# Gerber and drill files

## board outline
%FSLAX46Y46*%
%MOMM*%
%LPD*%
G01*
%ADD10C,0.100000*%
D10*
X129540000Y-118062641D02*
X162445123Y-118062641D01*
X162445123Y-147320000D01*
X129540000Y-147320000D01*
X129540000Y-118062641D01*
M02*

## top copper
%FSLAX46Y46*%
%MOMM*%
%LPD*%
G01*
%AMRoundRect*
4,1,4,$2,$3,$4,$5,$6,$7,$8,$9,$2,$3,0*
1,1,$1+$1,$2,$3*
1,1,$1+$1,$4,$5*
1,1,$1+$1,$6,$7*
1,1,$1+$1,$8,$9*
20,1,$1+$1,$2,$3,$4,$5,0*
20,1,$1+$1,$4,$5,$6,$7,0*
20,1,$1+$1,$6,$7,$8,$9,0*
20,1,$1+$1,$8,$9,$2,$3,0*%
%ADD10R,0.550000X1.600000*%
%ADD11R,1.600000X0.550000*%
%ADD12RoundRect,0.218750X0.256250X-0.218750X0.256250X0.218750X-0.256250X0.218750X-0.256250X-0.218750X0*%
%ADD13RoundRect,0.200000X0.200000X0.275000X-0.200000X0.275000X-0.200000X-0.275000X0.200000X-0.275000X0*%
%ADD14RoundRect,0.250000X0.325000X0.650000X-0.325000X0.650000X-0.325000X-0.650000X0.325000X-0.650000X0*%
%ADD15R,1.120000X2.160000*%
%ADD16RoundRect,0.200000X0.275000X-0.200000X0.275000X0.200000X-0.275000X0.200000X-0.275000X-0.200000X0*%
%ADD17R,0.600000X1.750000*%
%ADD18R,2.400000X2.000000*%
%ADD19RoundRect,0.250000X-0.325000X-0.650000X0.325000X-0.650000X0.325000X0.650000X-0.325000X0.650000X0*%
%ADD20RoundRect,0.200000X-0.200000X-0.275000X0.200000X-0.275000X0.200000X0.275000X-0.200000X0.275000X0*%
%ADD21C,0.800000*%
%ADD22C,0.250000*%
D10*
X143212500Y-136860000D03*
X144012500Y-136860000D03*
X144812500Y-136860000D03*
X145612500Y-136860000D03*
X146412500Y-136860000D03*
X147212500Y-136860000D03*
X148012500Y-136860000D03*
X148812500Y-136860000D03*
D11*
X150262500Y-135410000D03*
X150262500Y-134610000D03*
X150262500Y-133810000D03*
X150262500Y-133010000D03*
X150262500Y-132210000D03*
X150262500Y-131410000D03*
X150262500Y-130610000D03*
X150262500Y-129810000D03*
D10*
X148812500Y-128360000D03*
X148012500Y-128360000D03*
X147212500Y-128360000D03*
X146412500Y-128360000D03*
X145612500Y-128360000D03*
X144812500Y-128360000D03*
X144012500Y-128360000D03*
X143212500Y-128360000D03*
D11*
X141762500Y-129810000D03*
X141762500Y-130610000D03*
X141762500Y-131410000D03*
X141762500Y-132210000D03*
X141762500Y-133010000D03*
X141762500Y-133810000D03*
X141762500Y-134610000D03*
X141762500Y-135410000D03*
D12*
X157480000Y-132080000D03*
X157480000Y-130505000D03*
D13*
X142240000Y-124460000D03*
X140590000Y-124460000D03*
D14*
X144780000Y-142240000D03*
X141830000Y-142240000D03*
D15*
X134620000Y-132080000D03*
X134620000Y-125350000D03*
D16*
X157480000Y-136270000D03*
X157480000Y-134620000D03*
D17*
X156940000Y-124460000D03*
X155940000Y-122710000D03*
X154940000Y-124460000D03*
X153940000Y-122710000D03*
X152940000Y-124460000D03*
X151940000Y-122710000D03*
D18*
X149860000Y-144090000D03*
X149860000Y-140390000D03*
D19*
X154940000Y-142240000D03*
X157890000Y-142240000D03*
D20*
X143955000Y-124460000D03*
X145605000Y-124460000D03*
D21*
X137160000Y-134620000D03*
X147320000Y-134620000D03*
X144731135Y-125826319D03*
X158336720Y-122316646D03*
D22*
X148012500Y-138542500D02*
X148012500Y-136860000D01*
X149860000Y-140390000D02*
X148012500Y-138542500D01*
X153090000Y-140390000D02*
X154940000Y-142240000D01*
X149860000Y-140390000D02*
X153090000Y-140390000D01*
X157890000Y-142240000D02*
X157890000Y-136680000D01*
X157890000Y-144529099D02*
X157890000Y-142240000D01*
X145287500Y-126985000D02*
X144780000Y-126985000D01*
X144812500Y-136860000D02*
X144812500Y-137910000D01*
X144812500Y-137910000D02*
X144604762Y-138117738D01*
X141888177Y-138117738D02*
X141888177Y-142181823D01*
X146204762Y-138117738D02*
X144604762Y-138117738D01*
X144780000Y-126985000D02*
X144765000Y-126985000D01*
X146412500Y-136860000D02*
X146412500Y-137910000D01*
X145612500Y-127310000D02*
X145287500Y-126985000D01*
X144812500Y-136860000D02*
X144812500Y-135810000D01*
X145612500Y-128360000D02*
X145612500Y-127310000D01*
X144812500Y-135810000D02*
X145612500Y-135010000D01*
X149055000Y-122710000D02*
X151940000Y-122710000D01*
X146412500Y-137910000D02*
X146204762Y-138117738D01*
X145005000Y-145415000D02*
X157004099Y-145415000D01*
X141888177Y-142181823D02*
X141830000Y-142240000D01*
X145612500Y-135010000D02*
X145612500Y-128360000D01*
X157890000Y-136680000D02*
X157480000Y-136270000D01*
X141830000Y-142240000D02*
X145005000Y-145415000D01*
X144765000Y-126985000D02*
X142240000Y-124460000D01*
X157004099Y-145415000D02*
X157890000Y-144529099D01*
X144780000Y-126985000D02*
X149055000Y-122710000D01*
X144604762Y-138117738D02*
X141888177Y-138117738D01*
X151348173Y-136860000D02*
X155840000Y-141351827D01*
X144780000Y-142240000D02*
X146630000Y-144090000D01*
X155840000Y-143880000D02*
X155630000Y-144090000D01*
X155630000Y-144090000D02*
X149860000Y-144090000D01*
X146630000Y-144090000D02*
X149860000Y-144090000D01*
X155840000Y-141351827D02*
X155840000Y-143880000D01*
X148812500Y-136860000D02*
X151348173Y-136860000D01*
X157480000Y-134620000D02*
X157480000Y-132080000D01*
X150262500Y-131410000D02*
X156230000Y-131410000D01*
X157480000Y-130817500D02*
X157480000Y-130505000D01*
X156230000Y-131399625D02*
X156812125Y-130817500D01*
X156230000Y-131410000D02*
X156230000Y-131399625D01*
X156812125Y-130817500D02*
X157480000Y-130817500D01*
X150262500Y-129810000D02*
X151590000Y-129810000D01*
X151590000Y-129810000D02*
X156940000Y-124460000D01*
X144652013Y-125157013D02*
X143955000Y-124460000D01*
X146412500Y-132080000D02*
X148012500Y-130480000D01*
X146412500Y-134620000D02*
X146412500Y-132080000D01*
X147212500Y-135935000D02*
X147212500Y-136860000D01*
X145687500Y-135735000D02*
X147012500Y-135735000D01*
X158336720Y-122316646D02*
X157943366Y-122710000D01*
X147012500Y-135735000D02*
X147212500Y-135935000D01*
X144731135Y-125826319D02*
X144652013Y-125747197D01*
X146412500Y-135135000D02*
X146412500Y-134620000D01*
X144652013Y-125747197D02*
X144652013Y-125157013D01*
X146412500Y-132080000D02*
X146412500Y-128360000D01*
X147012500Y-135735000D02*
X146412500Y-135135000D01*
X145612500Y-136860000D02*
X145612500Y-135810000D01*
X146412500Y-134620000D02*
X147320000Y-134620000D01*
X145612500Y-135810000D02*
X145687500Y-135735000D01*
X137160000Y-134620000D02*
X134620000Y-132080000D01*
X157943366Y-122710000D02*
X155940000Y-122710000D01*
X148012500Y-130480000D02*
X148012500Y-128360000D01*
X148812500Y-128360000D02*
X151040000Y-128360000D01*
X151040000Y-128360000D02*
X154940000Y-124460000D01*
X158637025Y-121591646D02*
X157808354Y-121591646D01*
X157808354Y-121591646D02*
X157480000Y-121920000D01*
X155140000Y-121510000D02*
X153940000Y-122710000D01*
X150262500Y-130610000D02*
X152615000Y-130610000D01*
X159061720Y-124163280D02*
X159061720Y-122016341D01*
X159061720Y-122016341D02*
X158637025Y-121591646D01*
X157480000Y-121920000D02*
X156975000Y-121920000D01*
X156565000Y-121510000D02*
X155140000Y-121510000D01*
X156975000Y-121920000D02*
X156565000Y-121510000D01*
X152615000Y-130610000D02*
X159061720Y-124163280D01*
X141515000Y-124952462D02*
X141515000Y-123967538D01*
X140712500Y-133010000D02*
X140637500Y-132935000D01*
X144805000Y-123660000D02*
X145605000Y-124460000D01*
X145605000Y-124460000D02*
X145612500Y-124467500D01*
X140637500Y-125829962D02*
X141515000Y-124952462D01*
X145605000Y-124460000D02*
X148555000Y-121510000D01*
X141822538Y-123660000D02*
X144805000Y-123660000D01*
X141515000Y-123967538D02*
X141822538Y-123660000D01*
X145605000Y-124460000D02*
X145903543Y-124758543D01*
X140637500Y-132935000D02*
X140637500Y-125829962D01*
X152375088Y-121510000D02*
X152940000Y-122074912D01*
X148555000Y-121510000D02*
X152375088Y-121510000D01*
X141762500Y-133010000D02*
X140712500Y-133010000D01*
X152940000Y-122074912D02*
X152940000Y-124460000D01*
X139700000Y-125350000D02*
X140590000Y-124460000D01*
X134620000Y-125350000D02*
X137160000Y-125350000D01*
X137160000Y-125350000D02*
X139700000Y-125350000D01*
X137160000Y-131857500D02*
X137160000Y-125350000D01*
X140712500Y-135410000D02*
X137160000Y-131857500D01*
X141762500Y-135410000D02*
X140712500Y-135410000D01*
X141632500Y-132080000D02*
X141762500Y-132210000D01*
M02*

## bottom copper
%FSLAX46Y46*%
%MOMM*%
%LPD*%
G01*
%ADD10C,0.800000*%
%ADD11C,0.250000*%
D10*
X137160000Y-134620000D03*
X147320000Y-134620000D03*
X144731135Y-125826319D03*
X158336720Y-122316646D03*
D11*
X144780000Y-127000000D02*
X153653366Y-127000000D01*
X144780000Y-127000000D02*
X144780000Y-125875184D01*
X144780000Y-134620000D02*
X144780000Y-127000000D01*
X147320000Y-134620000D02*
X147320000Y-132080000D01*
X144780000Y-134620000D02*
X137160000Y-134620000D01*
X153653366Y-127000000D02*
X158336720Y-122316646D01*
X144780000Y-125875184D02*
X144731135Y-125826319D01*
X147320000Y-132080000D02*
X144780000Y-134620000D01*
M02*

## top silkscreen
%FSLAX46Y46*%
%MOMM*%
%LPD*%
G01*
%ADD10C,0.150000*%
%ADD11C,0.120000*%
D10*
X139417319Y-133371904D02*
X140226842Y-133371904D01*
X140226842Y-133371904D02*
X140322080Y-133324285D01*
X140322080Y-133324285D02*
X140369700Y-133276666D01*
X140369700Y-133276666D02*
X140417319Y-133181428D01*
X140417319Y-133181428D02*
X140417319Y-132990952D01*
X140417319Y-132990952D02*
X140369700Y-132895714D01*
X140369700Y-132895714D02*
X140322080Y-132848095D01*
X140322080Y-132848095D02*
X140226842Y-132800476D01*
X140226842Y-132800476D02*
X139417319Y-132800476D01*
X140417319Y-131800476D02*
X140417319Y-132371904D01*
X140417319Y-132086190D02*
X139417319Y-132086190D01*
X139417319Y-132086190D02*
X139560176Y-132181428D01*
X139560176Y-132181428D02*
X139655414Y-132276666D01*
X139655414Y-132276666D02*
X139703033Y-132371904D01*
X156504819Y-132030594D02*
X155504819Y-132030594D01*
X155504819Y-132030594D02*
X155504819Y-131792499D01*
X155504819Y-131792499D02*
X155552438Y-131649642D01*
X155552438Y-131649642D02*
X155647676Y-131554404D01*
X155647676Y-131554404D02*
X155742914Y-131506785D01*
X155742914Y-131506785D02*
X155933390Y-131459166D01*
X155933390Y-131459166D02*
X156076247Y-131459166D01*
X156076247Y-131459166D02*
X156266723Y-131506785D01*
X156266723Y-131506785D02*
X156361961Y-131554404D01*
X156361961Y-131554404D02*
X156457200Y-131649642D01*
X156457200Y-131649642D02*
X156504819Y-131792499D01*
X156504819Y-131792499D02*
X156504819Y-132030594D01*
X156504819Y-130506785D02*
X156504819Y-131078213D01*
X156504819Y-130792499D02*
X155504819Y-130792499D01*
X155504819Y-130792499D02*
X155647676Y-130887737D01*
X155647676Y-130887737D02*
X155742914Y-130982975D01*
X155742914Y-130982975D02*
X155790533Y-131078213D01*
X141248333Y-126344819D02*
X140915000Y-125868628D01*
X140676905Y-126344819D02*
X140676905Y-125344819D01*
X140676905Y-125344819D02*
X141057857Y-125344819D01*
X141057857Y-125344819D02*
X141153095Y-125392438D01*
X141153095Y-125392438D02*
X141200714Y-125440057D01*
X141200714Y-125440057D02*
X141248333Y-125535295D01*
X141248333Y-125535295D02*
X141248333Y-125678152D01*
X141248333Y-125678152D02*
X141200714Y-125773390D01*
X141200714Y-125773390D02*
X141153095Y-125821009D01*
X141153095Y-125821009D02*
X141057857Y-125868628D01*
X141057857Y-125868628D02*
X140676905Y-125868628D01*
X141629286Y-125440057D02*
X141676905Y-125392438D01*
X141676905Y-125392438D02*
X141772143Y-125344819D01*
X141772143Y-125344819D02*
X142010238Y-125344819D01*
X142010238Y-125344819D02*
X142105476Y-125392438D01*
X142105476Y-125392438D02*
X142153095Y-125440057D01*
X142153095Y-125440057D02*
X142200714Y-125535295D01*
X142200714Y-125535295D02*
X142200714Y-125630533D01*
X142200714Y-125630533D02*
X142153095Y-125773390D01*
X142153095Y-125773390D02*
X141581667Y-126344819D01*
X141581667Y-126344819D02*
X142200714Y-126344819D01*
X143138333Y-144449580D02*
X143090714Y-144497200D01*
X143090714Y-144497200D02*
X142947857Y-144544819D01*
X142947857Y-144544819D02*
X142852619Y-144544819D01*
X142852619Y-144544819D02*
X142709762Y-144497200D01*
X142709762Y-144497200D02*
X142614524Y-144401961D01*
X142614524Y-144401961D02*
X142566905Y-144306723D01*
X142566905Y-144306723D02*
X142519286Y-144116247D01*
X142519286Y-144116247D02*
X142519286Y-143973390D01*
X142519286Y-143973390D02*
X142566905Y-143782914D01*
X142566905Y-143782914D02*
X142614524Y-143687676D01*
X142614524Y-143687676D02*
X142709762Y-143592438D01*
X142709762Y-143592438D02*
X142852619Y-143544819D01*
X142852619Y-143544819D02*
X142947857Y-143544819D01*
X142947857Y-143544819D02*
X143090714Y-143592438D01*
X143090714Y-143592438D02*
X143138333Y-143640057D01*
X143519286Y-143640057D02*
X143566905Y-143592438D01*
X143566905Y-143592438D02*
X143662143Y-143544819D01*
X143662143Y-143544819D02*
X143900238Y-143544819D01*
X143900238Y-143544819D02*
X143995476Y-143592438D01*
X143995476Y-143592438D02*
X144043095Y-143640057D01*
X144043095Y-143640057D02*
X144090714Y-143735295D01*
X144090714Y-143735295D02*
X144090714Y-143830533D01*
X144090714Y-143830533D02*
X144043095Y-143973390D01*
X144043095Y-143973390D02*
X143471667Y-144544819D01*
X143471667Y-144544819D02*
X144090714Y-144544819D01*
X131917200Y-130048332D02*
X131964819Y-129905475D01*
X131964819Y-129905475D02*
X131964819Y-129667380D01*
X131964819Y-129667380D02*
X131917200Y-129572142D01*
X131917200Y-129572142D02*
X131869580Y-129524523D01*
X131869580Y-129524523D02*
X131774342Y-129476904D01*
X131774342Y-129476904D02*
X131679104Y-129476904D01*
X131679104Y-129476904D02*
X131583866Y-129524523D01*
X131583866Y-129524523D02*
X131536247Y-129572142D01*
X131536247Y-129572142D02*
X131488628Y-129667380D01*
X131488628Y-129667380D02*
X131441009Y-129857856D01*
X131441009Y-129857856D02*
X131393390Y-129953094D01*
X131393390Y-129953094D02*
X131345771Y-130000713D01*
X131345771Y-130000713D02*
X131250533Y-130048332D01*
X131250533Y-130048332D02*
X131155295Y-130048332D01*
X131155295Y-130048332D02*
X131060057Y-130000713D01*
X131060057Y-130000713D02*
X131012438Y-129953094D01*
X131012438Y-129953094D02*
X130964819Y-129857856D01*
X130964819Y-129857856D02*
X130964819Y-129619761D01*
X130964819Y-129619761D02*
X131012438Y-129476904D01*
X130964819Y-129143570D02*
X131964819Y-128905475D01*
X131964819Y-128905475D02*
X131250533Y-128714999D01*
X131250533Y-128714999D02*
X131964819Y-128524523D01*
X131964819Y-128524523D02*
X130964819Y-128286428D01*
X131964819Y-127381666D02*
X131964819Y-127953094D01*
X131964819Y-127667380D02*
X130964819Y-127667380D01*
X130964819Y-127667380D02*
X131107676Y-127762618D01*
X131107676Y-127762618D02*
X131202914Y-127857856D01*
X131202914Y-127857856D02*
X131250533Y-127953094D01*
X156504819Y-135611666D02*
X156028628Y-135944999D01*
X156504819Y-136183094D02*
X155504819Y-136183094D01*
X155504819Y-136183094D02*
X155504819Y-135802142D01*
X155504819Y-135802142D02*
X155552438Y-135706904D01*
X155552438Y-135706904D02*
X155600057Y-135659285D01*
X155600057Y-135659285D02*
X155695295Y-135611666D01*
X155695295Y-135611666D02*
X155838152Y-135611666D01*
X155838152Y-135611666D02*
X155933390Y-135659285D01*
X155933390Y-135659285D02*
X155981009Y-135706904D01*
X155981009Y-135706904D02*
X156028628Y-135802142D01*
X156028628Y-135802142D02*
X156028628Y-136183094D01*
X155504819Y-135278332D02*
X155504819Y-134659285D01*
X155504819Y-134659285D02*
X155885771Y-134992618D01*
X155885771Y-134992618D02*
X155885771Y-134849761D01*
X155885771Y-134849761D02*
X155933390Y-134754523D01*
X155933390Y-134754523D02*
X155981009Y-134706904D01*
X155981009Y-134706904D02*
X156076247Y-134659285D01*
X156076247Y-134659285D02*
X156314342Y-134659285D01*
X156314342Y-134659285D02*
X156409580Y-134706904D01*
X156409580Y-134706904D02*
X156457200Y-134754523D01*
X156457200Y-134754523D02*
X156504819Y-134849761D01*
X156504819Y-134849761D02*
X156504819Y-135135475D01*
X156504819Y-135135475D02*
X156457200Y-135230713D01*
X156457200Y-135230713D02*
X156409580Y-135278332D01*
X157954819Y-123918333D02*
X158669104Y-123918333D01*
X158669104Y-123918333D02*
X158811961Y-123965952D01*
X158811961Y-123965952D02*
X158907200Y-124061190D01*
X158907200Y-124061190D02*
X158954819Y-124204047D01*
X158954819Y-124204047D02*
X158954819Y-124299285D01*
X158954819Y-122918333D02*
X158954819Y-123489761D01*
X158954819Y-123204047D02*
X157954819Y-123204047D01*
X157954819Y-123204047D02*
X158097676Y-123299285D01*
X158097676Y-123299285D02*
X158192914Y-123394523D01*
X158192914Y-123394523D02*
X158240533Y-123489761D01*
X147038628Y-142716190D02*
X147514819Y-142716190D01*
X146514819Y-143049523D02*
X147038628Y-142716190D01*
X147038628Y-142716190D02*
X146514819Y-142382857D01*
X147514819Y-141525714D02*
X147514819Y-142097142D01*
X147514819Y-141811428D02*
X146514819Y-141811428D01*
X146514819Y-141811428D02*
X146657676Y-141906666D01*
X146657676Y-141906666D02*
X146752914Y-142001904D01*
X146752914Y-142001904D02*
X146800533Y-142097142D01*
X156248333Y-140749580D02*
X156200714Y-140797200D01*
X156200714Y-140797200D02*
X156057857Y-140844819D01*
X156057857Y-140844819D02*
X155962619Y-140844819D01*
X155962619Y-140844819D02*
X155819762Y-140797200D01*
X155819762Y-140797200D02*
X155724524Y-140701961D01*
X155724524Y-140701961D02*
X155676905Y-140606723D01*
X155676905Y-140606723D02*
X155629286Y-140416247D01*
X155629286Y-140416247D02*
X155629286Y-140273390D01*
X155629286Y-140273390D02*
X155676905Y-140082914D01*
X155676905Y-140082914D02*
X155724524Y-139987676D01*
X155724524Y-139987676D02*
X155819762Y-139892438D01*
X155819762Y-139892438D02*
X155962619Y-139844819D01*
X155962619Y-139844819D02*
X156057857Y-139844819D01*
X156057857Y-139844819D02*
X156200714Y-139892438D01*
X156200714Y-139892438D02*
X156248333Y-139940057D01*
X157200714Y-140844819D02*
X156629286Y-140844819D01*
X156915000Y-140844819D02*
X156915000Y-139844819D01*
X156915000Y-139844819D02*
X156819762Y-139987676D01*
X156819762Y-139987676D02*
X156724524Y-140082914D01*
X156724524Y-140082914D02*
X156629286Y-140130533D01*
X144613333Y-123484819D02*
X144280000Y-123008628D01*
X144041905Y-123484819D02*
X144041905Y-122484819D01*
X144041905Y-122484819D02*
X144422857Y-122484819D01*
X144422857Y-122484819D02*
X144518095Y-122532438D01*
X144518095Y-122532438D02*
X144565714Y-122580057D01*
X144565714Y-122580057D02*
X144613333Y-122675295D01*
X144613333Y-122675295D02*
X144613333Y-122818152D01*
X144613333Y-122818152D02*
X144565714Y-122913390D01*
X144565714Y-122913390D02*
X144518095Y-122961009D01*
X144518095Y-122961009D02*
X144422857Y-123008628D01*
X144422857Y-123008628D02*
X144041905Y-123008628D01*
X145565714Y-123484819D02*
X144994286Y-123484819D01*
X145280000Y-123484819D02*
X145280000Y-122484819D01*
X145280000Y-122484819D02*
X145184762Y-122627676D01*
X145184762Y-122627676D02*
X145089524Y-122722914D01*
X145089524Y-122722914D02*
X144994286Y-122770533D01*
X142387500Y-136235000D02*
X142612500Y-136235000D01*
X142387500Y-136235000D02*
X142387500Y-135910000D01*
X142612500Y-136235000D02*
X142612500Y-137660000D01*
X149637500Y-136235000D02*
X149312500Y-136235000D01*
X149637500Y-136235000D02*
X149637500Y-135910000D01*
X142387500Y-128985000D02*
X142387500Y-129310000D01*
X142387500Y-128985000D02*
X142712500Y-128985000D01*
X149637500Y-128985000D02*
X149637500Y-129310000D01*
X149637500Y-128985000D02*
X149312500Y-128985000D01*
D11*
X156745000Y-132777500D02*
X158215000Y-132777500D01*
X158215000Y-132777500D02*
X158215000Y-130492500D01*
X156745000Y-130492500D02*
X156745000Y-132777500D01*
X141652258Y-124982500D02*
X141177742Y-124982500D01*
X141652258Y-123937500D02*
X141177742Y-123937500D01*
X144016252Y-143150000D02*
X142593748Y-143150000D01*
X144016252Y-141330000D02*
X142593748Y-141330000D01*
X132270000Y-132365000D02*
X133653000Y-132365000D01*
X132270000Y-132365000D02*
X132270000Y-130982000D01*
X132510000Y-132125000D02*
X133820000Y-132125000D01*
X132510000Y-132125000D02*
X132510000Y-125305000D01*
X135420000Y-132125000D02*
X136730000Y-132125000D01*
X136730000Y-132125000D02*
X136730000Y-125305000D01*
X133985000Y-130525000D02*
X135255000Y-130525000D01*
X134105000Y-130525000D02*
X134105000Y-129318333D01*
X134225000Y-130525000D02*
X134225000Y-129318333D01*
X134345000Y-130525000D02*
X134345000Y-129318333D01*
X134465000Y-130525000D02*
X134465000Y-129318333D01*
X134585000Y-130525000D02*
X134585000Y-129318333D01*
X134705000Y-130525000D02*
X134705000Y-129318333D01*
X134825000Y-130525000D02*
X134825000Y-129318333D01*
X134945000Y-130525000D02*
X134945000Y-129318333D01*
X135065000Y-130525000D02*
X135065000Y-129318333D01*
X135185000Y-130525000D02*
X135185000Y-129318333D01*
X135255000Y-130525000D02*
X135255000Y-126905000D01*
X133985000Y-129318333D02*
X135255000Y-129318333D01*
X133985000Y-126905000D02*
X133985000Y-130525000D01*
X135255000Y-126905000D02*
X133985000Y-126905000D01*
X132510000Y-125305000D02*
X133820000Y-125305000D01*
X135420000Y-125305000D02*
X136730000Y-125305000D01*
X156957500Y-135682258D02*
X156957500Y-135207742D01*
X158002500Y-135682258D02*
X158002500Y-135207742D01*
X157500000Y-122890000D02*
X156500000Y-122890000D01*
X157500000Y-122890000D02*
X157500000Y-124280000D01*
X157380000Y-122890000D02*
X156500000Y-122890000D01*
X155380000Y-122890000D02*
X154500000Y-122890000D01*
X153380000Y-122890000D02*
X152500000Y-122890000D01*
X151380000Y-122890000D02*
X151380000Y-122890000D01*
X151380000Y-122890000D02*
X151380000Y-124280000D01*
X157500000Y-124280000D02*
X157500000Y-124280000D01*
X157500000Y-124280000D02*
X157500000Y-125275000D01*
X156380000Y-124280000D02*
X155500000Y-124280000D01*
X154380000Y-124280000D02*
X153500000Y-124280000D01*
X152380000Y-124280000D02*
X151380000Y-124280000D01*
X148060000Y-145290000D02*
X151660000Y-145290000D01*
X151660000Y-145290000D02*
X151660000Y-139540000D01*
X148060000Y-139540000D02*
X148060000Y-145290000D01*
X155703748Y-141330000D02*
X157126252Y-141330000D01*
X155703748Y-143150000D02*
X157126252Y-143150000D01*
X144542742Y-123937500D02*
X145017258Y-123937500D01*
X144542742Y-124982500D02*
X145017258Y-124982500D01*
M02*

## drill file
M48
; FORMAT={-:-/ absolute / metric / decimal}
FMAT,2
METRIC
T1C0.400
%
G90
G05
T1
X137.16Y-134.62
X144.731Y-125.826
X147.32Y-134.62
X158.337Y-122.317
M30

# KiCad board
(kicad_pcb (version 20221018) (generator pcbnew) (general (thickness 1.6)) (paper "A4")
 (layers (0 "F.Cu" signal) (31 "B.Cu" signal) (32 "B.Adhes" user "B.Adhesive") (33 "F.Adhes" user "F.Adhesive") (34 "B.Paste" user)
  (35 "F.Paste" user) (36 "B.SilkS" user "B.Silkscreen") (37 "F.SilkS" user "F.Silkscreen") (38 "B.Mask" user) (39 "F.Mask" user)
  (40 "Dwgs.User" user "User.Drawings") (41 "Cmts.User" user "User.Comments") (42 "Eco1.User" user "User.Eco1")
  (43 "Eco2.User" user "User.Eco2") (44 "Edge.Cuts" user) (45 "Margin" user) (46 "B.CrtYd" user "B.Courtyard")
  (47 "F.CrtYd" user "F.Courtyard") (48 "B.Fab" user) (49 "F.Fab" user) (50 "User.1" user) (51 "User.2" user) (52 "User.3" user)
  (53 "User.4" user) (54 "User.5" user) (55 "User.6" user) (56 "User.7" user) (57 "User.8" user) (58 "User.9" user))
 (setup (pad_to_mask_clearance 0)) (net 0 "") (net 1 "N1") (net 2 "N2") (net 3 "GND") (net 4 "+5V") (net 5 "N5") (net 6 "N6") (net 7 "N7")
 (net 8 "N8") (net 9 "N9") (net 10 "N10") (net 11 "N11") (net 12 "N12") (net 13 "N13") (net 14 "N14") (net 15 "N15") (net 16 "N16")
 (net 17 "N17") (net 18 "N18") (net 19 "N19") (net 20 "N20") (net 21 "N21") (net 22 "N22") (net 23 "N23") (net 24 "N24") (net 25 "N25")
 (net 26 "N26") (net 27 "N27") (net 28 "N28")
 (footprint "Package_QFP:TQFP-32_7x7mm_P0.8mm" (layer "F.Cu") (at 146.0125 132.61 90)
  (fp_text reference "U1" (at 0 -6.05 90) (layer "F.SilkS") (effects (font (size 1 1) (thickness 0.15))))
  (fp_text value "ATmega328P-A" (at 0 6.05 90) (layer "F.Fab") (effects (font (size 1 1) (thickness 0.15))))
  (fp_line (start -3.625 -3.625) (end -3.625 -3.4) (stroke (width 0.15) (type solid)) (layer "F.SilkS"))
  (fp_line (start -3.625 -3.625) (end -3.3 -3.625) (stroke (width 0.15) (type solid)) (layer "F.SilkS"))
  (fp_line (start -3.625 -3.4) (end -5.05 -3.4) (stroke (width 0.15) (type solid)) (layer "F.SilkS"))
  (fp_line (start -3.625 3.625) (end -3.625 3.3) (stroke (width 0.15) (type solid)) (layer "F.SilkS"))
  (fp_line (start -3.625 3.625) (end -3.3 3.625) (stroke (width 0.15) (type solid)) (layer "F.SilkS"))
  (fp_line (start 3.625 -3.625) (end 3.3 -3.625) (stroke (width 0.15) (type solid)) (layer "F.SilkS"))
  (fp_line (start 3.625 -3.625) (end 3.625 -3.3) (stroke (width 0.15) (type solid)) (layer "F.SilkS"))
  (fp_line (start 3.625 3.625) (end 3.3 3.625) (stroke (width 0.15) (type solid)) (layer "F.SilkS"))
  (fp_line (start 3.625 3.625) (end 3.625 3.3) (stroke (width 0.15) (type solid)) (layer "F.SilkS"))
  (pad "1" smd rect (at -4.25 -2.8 90) (size 1.6 0.55) (layers "F.Cu" "F.Paste" "F.Mask") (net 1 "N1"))
  (pad "2" smd rect (at -4.25 -2 90) (size 1.6 0.55) (layers "F.Cu" "F.Paste" "F.Mask") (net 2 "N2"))
  (pad "3" smd rect (at -4.25 -1.2 90) (size 1.6 0.55) (layers "F.Cu" "F.Paste" "F.Mask") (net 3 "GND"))
  (pad "4" smd rect (at -4.25 -0.4 90) (size 1.6 0.55) (layers "F.Cu" "F.Paste" "F.Mask") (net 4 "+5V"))
  (pad "5" smd rect (at -4.25 0.4 90) (size 1.6 0.55) (layers "F.Cu" "F.Paste" "F.Mask") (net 3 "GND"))
  (pad "6" smd rect (at -4.25 1.2 90) (size 1.6 0.55) (layers "F.Cu" "F.Paste" "F.Mask") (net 4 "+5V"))
  (pad "7" smd rect (at -4.25 2 90) (size 1.6 0.55) (layers "F.Cu" "F.Paste" "F.Mask") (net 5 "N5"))
  (pad "8" smd rect (at -4.25 2.8 90) (size 1.6 0.55) (layers "F.Cu" "F.Paste" "F.Mask") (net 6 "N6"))
  (pad "9" smd rect (at -2.8 4.25 180) (size 1.6 0.55) (layers "F.Cu" "F.Paste" "F.Mask") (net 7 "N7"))
  (pad "10" smd rect (at -2 4.25 180) (size 1.6 0.55) (layers "F.Cu" "F.Paste" "F.Mask") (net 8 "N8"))
  (pad "11" smd rect (at -1.2 4.25 180) (size 1.6 0.55) (layers "F.Cu" "F.Paste" "F.Mask") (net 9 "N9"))
  (pad "12" smd rect (at -0.4 4.25 180) (size 1.6 0.55) (layers "F.Cu" "F.Paste" "F.Mask") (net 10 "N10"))
  (pad "13" smd rect (at 0.4 4.25 180) (size 1.6 0.55) (layers "F.Cu" "F.Paste" "F.Mask") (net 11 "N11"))
  (pad "14" smd rect (at 1.2 4.25 180) (size 1.6 0.55) (layers "F.Cu" "F.Paste" "F.Mask") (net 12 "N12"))
  (pad "15" smd rect (at 2 4.25 180) (size 1.6 0.55) (layers "F.Cu" "F.Paste" "F.Mask") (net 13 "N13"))
  (pad "16" smd rect (at 2.8 4.25 180) (size 1.6 0.55) (layers "F.Cu" "F.Paste" "F.Mask") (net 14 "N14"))
  (pad "17" smd rect (at 4.25 2.8 90) (size 1.6 0.55) (layers "F.Cu" "F.Paste" "F.Mask") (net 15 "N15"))
  (pad "18" smd rect (at 4.25 2 90) (size 1.6 0.55) (layers "F.Cu" "F.Paste" "F.Mask") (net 4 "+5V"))
  (pad "19" smd rect (at 4.25 1.2 90) (size 1.6 0.55) (layers "F.Cu" "F.Paste" "F.Mask") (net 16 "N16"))
  (pad "20" smd rect (at 4.25 0.4 90) (size 1.6 0.55) (layers "F.Cu" "F.Paste" "F.Mask") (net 4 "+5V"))
  (pad "21" smd rect (at 4.25 -0.4 90) (size 1.6 0.55) (layers "F.Cu" "F.Paste" "F.Mask") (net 3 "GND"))
  (pad "22" smd rect (at 4.25 -1.2 90) (size 1.6 0.55) (layers "F.Cu" "F.Paste" "F.Mask") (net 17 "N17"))
  (pad "23" smd rect (at 4.25 -2 90) (size 1.6 0.55) (layers "F.Cu" "F.Paste" "F.Mask") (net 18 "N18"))
  (pad "24" smd rect (at 4.25 -2.8 90) (size 1.6 0.55) (layers "F.Cu" "F.Paste" "F.Mask") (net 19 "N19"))
  (pad "25" smd rect (at 2.8 -4.25 180) (size 1.6 0.55) (layers "F.Cu" "F.Paste" "F.Mask") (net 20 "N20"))
  (pad "26" smd rect (at 2 -4.25 180) (size 1.6 0.55) (layers "F.Cu" "F.Paste" "F.Mask") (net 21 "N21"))
  (pad "27" smd rect (at 1.2 -4.25 180) (size 1.6 0.55) (layers "F.Cu" "F.Paste" "F.Mask") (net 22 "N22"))
  (pad "28" smd rect (at 0.4 -4.25 180) (size 1.6 0.55) (layers "F.Cu" "F.Paste" "F.Mask") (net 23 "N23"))
  (pad "29" smd rect (at -0.4 -4.25 180) (size 1.6 0.55) (layers "F.Cu" "F.Paste" "F.Mask") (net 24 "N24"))
  (pad "30" smd rect (at -1.2 -4.25 180) (size 1.6 0.55) (layers "F.Cu" "F.Paste" "F.Mask") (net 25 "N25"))
  (pad "31" smd rect (at -2 -4.25 180) (size 1.6 0.55) (layers "F.Cu" "F.Paste" "F.Mask") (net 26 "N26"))
  (pad "32" smd rect (at -2.8 -4.25 180) (size 1.6 0.55) (layers "F.Cu" "F.Paste" "F.Mask") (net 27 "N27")))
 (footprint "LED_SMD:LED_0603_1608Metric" (layer "F.Cu") (at 157.48 131.2925 90)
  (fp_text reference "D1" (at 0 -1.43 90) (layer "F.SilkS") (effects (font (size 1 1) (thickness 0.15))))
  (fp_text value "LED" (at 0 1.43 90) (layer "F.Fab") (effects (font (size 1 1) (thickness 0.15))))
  (fp_line (start -1.485 -0.735) (end -1.485 0.735) (stroke (width 0.12) (type solid)) (layer "F.SilkS"))
  (fp_line (start -1.485 0.735) (end 0.8 0.735) (stroke (width 0.12) (type solid)) (layer "F.SilkS"))
  (fp_line (start 0.8 -0.735) (end -1.485 -0.735) (stroke (width 0.12) (type solid)) (layer "F.SilkS"))
  (pad "1" smd roundrect (at -0.7875 0 90) (size 0.875 0.95) (layers "F.Cu" "F.Paste" "F.Mask") (roundrect_rratio 0.25) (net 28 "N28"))
  (pad "2" smd roundrect (at 0.7875 0 90) (size 0.875 0.95) (layers "F.Cu" "F.Paste" "F.Mask") (roundrect_rratio 0.25) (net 12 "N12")))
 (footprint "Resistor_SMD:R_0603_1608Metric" (layer "F.Cu") (at 141.415 124.46 180)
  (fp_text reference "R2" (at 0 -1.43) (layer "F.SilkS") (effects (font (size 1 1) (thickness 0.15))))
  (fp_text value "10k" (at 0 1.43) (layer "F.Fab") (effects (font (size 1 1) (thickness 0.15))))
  (fp_line (start -0.237258 -0.5225) (end 0.237258 -0.5225) (stroke (width 0.12) (type solid)) (layer "F.SilkS"))
  (fp_line (start -0.237258 0.5225) (end 0.237258 0.5225) (stroke (width 0.12) (type solid)) (layer "F.SilkS"))
  (pad "1" smd roundrect (at -0.825 0 180) (size 0.8 0.95) (layers "F.Cu" "F.Paste" "F.Mask") (roundrect_rratio 0.25) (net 3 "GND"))
  (pad "2" smd roundrect (at 0.825 0 180) (size 0.8 0.95) (layers "F.Cu" "F.Paste" "F.Mask") (roundrect_rratio 0.25) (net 27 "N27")))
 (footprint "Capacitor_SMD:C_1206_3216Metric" (layer "F.Cu") (at 143.305 142.24 180)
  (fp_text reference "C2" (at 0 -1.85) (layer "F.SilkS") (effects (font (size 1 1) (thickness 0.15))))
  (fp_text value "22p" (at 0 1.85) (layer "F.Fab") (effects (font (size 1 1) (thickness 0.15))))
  (fp_line (start -0.711252 -0.91) (end 0.711252 -0.91) (stroke (width 0.12) (type solid)) (layer "F.SilkS"))
  (fp_line (start -0.711252 0.91) (end 0.711252 0.91) (stroke (width 0.12) (type solid)) (layer "F.SilkS"))
  (pad "1" smd roundrect (at -1.475 0 180) (size 1.15 1.8) (layers "F.Cu" "F.Paste" "F.Mask") (roundrect_rratio 0.2173913043) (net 6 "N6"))
  (pad "2" smd roundrect (at 1.475 0 180) (size 1.15 1.8) (layers "F.Cu" "F.Paste" "F.Mask") (roundrect_rratio 0.2173913043) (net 3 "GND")))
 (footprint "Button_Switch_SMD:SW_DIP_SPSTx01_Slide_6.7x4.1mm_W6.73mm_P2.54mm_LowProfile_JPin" (layer "F.Cu") (at 134.62 128.715 90)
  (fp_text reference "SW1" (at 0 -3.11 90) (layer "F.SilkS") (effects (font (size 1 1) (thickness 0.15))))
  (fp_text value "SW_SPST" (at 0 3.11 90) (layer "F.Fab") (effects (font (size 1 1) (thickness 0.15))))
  (fp_line (start -3.65 -2.35) (end -3.65 -0.967) (stroke (width 0.12) (type solid)) (layer "F.SilkS"))
  (fp_line (start -3.65 -2.35) (end -2.267 -2.35) (stroke (width 0.12) (type solid)) (layer "F.SilkS"))
  (fp_line (start -3.41 -2.11) (end -3.41 -0.8) (stroke (width 0.12) (type solid)) (layer "F.SilkS"))
  (fp_line (start -3.41 -2.11) (end 3.41 -2.11) (stroke (width 0.12) (type solid)) (layer "F.SilkS"))
  (fp_line (start -3.41 0.8) (end -3.41 2.11) (stroke (width 0.12) (type solid)) (layer "F.SilkS"))
  (fp_line (start -3.41 2.11) (end 3.41 2.11) (stroke (width 0.12) (type solid)) (layer "F.SilkS"))
  (fp_line (start -1.81 -0.635) (end -1.81 0.635) (stroke (width 0.12) (type solid)) (layer "F.SilkS"))
  (fp_line (start -1.81 -0.515) (end -0.603333 -0.515) (stroke (width 0.12) (type solid)) (layer "F.SilkS"))
  (fp_line (start -1.81 -0.395) (end -0.603333 -0.395) (stroke (width 0.12) (type solid)) (layer "F.SilkS"))
  (fp_line (start -1.81 -0.275) (end -0.603333 -0.275) (stroke (width 0.12) (type solid)) (layer "F.SilkS"))
  (fp_line (start -1.81 -0.155) (end -0.603333 -0.155) (stroke (width 0.12) (type solid)) (layer "F.SilkS"))
  (fp_line (start -1.81 -0.035) (end -0.603333 -0.035) (stroke (width 0.12) (type solid)) (layer "F.SilkS"))
  (fp_line (start -1.81 0.085) (end -0.603333 0.085) (stroke (width 0.12) (type solid)) (layer "F.SilkS"))
  (fp_line (start -1.81 0.205) (end -0.603333 0.205) (stroke (width 0.12) (type solid)) (layer "F.SilkS"))
  (fp_line (start -1.81 0.325) (end -0.603333 0.325) (stroke (width 0.12) (type solid)) (layer "F.SilkS"))
  (fp_line (start -1.81 0.445) (end -0.603333 0.445) (stroke (width 0.12) (type solid)) (layer "F.SilkS"))
  (fp_line (start -1.81 0.565) (end -0.603333 0.565) (stroke (width 0.12) (type solid)) (layer "F.SilkS"))
  (fp_line (start -1.81 0.635) (end 1.81 0.635) (stroke (width 0.12) (type solid)) (layer "F.SilkS"))
  (fp_line (start -0.603333 -0.635) (end -0.603333 0.635) (stroke (width 0.12) (type solid)) (layer "F.SilkS"))
  (fp_line (start 1.81 -0.635) (end -1.81 -0.635) (stroke (width 0.12) (type solid)) (layer "F.SilkS"))
  (fp_line (start 1.81 0.635) (end 1.81 -0.635) (stroke (width 0.12) (type solid)) (layer "F.SilkS"))
  (fp_line (start 3.41 -2.11) (end 3.41 -0.8) (stroke (width 0.12) (type solid)) (layer "F.SilkS"))
  (fp_line (start 3.41 0.8) (end 3.41 2.11) (stroke (width 0.12) (type solid)) (layer "F.SilkS"))
  (pad "1" smd rect (at -3.365 0 90) (size 2.16 1.12) (layers "F.Cu" "F.Paste" "F.Mask") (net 4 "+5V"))
  (pad "2" smd rect (at 3.365 0 90) (size 2.16 1.12) (layers "F.Cu" "F.Paste" "F.Mask") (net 27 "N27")))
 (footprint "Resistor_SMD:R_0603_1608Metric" (layer "F.Cu") (at 157.48 135.445 90)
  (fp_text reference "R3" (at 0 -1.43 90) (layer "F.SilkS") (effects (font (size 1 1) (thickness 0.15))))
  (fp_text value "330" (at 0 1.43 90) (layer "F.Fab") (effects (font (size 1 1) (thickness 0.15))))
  (fp_line (start -0.237258 -0.5225) (end 0.237258 -0.5225) (stroke (width 0.12) (type solid)) (layer "F.SilkS"))
  (fp_line (start -0.237258 0.5225) (end 0.237258 0.5225) (stroke (width 0.12) (type solid)) (layer "F.SilkS"))
  (pad "1" smd roundrect (at -0.825 0 90) (size 0.8 0.95) (layers "F.Cu" "F.Paste" "F.Mask") (roundrect_rratio 0.25) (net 3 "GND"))
  (pad "2" smd roundrect (at 0.825 0 90) (size 0.8 0.95) (layers "F.Cu" "F.Paste" "F.Mask") (roundrect_rratio 0.25) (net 28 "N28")))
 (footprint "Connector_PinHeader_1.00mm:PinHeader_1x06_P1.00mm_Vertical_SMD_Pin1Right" (layer "F.Cu") (at 154.44 123.585 -90)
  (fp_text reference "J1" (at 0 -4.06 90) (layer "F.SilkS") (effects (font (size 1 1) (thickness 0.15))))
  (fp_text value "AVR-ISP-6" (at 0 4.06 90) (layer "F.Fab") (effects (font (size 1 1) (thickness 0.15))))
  (fp_line (start -0.695 -3.06) (end -0.695 -2.06) (stroke (width 0.12) (type solid)) (layer "F.SilkS"))
  (fp_line (start -0.695 -3.06) (end 0.695 -3.06) (stroke (width 0.12) (type solid)) (layer "F.SilkS"))
  (fp_line (start -0.695 -2.94) (end -0.695 -2.06) (stroke (width 0.12) (type solid)) (layer "F.SilkS"))
  (fp_line (start -0.695 -0.94) (end -0.695 -0.06) (stroke (width 0.12) (type solid)) (layer "F.SilkS"))
  (fp_line (start -0.695 1.06) (end -0.695 1.94) (stroke (width 0.12) (type solid)) (layer "F.SilkS"))
  (fp_line (start -0.695 3.06) (end -0.695 3.06) (stroke (width 0.12) (type solid)) (layer "F.SilkS"))
  (fp_line (start -0.695 3.06) (end 0.695 3.06) (stroke (width 0.12) (type solid)) (layer "F.SilkS"))
  (fp_line (start 0.695 -3.06) (end 0.695 -3.06) (stroke (width 0.12) (type solid)) (layer "F.SilkS"))
  (fp_line (start 0.695 -3.06) (end 1.69 -3.06) (stroke (width 0.12) (type solid)) (layer "F.SilkS"))
  (fp_line (start 0.695 -1.94) (end 0.695 -1.06) (stroke (width 0.12) (type solid)) (layer "F.SilkS"))
  (fp_line (start 0.695 0.06) (end 0.695 0.94) (stroke (width 0.12) (type solid)) (layer "F.SilkS"))
  (fp_line (start 0.695 2.06) (end 0.695 3.06) (stroke (width 0.12) (type solid)) (layer "F.SilkS"))
  (pad "1" smd rect (at 0.875 -2.5 270) (size 1.75 0.6) (layers "F.Cu" "F.Paste" "F.Mask") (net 14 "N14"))
  (pad "2" smd rect (at -0.875 -1.5 270) (size 1.75 0.6) (layers "F.Cu" "F.Paste" "F.Mask") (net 4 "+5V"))
  (pad "3" smd rect (at 0.875 -0.5 270) (size 1.75 0.6) (layers "F.Cu" "F.Paste" "F.Mask") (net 15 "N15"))
  (pad "4" smd rect (at -0.875 0.5 270) (size 1.75 0.6) (layers "F.Cu" "F.Paste" "F.Mask") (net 13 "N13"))
  (pad "5" smd rect (at 0.875 1.5 270) (size 1.75 0.6) (layers "F.Cu" "F.Paste" "F.Mask") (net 24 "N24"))
  (pad "6" smd rect (at -0.875 2.5 270) (size 1.75 0.6) (layers "F.Cu" "F.Paste" "F.Mask") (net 3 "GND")))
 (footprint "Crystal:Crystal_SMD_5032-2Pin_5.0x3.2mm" (layer "F.Cu") (at 149.86 142.24 90)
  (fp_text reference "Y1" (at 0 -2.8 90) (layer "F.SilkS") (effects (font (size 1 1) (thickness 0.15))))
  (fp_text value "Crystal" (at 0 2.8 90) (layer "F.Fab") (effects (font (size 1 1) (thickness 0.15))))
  (fp_line (start -3.05 -1.8) (end -3.05 1.8) (stroke (width 0.12) (type solid)) (layer "F.SilkS"))
  (fp_line (start -3.05 1.8) (end 2.7 1.8) (stroke (width 0.12) (type solid)) (layer "F.SilkS"))
  (fp_line (start 2.7 -1.8) (end -3.05 -1.8) (stroke (width 0.12) (type solid)) (layer "F.SilkS"))
  (pad "1" smd rect (at -1.85 0 90) (size 2 2.4) (layers "F.Cu" "F.Paste" "F.Mask") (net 6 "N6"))
  (pad "2" smd rect (at 1.85 0 90) (size 2 2.4) (layers "F.Cu" "F.Paste" "F.Mask") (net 5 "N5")))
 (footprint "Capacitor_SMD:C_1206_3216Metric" (layer "F.Cu") (at 156.415 142.24)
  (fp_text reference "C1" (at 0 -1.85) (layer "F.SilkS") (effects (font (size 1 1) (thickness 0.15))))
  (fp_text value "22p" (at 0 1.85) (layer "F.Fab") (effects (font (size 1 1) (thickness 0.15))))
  (fp_line (start -0.711252 -0.91) (end 0.711252 -0.91) (stroke (width 0.12) (type solid)) (layer "F.SilkS"))
  (fp_line (start -0.711252 0.91) (end 0.711252 0.91) (stroke (width 0.12) (type solid)) (layer "F.SilkS"))
  (pad "1" smd roundrect (at -1.475 0) (size 1.15 1.8) (layers "F.Cu" "F.Paste" "F.Mask") (roundrect_rratio 0.2173913043) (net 5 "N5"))
  (pad "2" smd roundrect (at 1.475 0) (size 1.15 1.8) (layers "F.Cu" "F.Paste" "F.Mask") (roundrect_rratio 0.2173913043) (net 3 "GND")))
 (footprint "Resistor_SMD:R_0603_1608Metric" (layer "F.Cu") (at 144.78 124.46)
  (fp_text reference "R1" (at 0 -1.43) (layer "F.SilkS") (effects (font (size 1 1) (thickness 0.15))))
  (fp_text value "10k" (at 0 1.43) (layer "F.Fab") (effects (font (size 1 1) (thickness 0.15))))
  (fp_line (start -0.237258 -0.5225) (end 0.237258 -0.5225) (stroke (width 0.12) (type solid)) (layer "F.SilkS"))
  (fp_line (start -0.237258 0.5225) (end 0.237258 0.5225) (stroke (width 0.12) (type solid)) (layer "F.SilkS"))
  (pad "1" smd roundrect (at -0.825 0) (size 0.8 0.95) (layers "F.Cu" "F.Paste" "F.Mask") (roundrect_rratio 0.25) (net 4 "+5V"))
  (pad "2" smd roundrect (at 0.825 0) (size 0.8 0.95) (layers "F.Cu" "F.Paste" "F.Mask") (roundrect_rratio 0.25) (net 24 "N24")))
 (gr_rect (start 129.54 118.062641) (end 162.445123 147.32) (stroke (width 0.1) (type default)) (fill none) (layer "Edge.Cuts"))
 (segment (start 148.0125 138.5425) (end 148.0125 136.86) (width 0.25) (layer "F.Cu") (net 5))
 (segment (start 149.86 140.39) (end 148.0125 138.5425) (width 0.25) (layer "F.Cu") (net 5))
 (segment (start 153.09 140.39) (end 154.94 142.24) (width 0.25) (layer "F.Cu") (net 5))
 (segment (start 149.86 140.39) (end 153.09 140.39) (width 0.25) (layer "F.Cu") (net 5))
 (segment (start 157.89 142.24) (end 157.89 136.68) (width 0.25) (layer "F.Cu") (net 3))
 (segment (start 157.89 144.529099) (end 157.89 142.24) (width 0.25) (layer "F.Cu") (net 3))
 (segment (start 145.2875 126.985) (end 144.78 126.985) (width 0.25) (layer "F.Cu") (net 3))
 (segment (start 144.8125 136.86) (end 144.8125 137.91) (width 0.25) (layer "F.Cu") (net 3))
 (segment (start 144.8125 137.91) (end 144.604762 138.117738) (width 0.25) (layer "F.Cu") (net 3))
 (segment (start 141.888177 138.117738) (end 141.888177 142.181823) (width 0.25) (layer "F.Cu") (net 3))
 (segment (start 146.204762 138.117738) (end 144.604762 138.117738) (width 0.25) (layer "F.Cu") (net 3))
 (segment (start 144.78 126.985) (end 144.765 126.985) (width 0.25) (layer "F.Cu") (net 3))
 (segment (start 146.4125 136.86) (end 146.4125 137.91) (width 0.25) (layer "F.Cu") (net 3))
 (segment (start 145.6125 127.31) (end 145.2875 126.985) (width 0.25) (layer "F.Cu") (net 3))
 (segment (start 144.8125 136.86) (end 144.8125 135.81) (width 0.25) (layer "F.Cu") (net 3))
 (segment (start 145.6125 128.36) (end 145.6125 127.31) (width 0.25) (layer "F.Cu") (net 3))
 (segment (start 144.8125 135.81) (end 145.6125 135.01) (width 0.25) (layer "F.Cu") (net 3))
 (segment (start 149.055 122.71) (end 151.94 122.71) (width 0.25) (layer "F.Cu") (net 3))
 (segment (start 146.4125 137.91) (end 146.204762 138.117738) (width 0.25) (layer "F.Cu") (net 3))
 (segment (start 145.005 145.415) (end 157.004099 145.415) (width 0.25) (layer "F.Cu") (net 3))
 (segment (start 141.888177 142.181823) (end 141.83 142.24) (width 0.25) (layer "F.Cu") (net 3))
 (segment (start 145.6125 135.01) (end 145.6125 128.36) (width 0.25) (layer "F.Cu") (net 3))
 (segment (start 157.89 136.68) (end 157.48 136.27) (width 0.25) (layer "F.Cu") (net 3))
 (segment (start 141.83 142.24) (end 145.005 145.415) (width 0.25) (layer "F.Cu") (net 3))
 (segment (start 144.765 126.985) (end 142.24 124.46) (width 0.25) (layer "F.Cu") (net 3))
 (segment (start 157.004099 145.415) (end 157.89 144.529099) (width 0.25) (layer "F.Cu") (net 3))
 (segment (start 144.78 126.985) (end 149.055 122.71) (width 0.25) (layer "F.Cu") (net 3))
 (segment (start 144.604762 138.117738) (end 141.888177 138.117738) (width 0.25) (layer "F.Cu") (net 3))
 (segment (start 151.348173 136.86) (end 155.84 141.351827) (width 0.25) (layer "F.Cu") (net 6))
 (segment (start 144.78 142.24) (end 146.63 144.09) (width 0.25) (layer "F.Cu") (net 6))
 (segment (start 155.84 143.88) (end 155.63 144.09) (width 0.25) (layer "F.Cu") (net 6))
 (segment (start 155.63 144.09) (end 149.86 144.09) (width 0.25) (layer "F.Cu") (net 6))
 (segment (start 146.63 144.09) (end 149.86 144.09) (width 0.25) (layer "F.Cu") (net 6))
 (segment (start 155.84 141.351827) (end 155.84 143.88) (width 0.25) (layer "F.Cu") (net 6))
 (segment (start 148.8125 136.86) (end 151.348173 136.86) (width 0.25) (layer "F.Cu") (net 6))
 (segment (start 157.48 134.62) (end 157.48 132.08) (width 0.25) (layer "F.Cu") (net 28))
 (segment (start 150.2625 131.41) (end 156.23 131.41) (width 0.25) (layer "F.Cu") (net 12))
 (segment (start 157.48 130.8175) (end 157.48 130.505) (width 0.25) (layer "F.Cu") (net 12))
 (segment (start 156.23 131.399625) (end 156.812125 130.8175) (width 0.25) (layer "F.Cu") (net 12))
 (segment (start 156.23 131.41) (end 156.23 131.399625) (width 0.25) (layer "F.Cu") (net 12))
 (segment (start 156.812125 130.8175) (end 157.48 130.8175) (width 0.25) (layer "F.Cu") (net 12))
 (segment (start 150.2625 129.81) (end 151.59 129.81) (width 0.25) (layer "F.Cu") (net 14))
 (segment (start 151.59 129.81) (end 156.94 124.46) (width 0.25) (layer "F.Cu") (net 14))
 (segment (start 144.652013 125.157013) (end 143.955 124.46) (width 0.25) (layer "F.Cu") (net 4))
 (segment (start 146.4125 132.08) (end 148.0125 130.48) (width 0.25) (layer "F.Cu") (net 4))
 (segment (start 146.4125 134.62) (end 146.4125 132.08) (width 0.25) (layer "F.Cu") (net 4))
 (segment (start 147.2125 135.935) (end 147.2125 136.86) (width 0.25) (layer "F.Cu") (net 4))
 (segment (start 145.6875 135.735) (end 147.0125 135.735) (width 0.25) (layer "F.Cu") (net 4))
 (segment (start 158.33672 122.316646) (end 157.943366 122.71) (width 0.25) (layer "F.Cu") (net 4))
 (segment (start 147.0125 135.735) (end 147.2125 135.935) (width 0.25) (layer "F.Cu") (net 4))
 (segment (start 144.731135 125.826319) (end 144.652013 125.747197) (width 0.25) (layer "F.Cu") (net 4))
 (segment (start 146.4125 135.135) (end 146.4125 134.62) (width 0.25) (layer "F.Cu") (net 4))
 (segment (start 144.652013 125.747197) (end 144.652013 125.157013) (width 0.25) (layer "F.Cu") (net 4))
 (segment (start 146.4125 132.08) (end 146.4125 128.36) (width 0.25) (layer "F.Cu") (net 4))
 (segment (start 147.0125 135.735) (end 146.4125 135.135) (width 0.25) (layer "F.Cu") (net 4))
 (segment (start 145.6125 136.86) (end 145.6125 135.81) (width 0.25) (layer "F.Cu") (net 4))
 (segment (start 146.4125 134.62) (end 147.32 134.62) (width 0.25) (layer "F.Cu") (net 4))
 (segment (start 145.6125 135.81) (end 145.6875 135.735) (width 0.25) (layer "F.Cu") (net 4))
 (segment (start 137.16 134.62) (end 134.62 132.08) (width 0.25) (layer "F.Cu") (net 4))
 (segment (start 157.943366 122.71) (end 155.94 122.71) (width 0.25) (layer "F.Cu") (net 4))
 (segment (start 148.0125 130.48) (end 148.0125 128.36) (width 0.25) (layer "F.Cu") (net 4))
 (via (at 137.16 134.62) (size 0.8) (drill 0.4) (layers "F.Cu" "B.Cu") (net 4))
 (via (at 147.32 134.62) (size 0.8) (drill 0.4) (layers "F.Cu" "B.Cu") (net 4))
 (via (at 144.731135 125.826319) (size 0.8) (drill 0.4) (layers "F.Cu" "B.Cu") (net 4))
 (via (at 158.33672 122.316646) (size 0.8) (drill 0.4) (layers "F.Cu" "B.Cu") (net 4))
 (segment (start 144.78 127) (end 153.653366 127) (width 0.25) (layer "B.Cu") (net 4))
 (segment (start 144.78 127) (end 144.78 125.875184) (width 0.25) (layer "B.Cu") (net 4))
 (segment (start 144.78 134.62) (end 144.78 127) (width 0.25) (layer "B.Cu") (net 4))
 (segment (start 147.32 134.62) (end 147.32 132.08) (width 0.25) (layer "B.Cu") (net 4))
 (segment (start 144.78 134.62) (end 137.16 134.62) (width 0.25) (layer "B.Cu") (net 4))
 (segment (start 153.653366 127) (end 158.33672 122.316646) (width 0.25) (layer "B.Cu") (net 4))
 (segment (start 144.78 125.875184) (end 144.731135 125.826319) (width 0.25) (layer "B.Cu") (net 4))
 (segment (start 147.32 132.08) (end 144.78 134.62) (width 0.25) (layer "B.Cu") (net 4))
 (segment (start 148.8125 128.36) (end 151.04 128.36) (width 0.25) (layer "F.Cu") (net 15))
 (segment (start 151.04 128.36) (end 154.94 124.46) (width 0.25) (layer "F.Cu") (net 15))
 (segment (start 158.637025 121.591646) (end 157.808354 121.591646) (width 0.25) (layer "F.Cu") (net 13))
 (segment (start 157.808354 121.591646) (end 157.48 121.92) (width 0.25) (layer "F.Cu") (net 13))
 (segment (start 155.14 121.51) (end 153.94 122.71) (width 0.25) (layer "F.Cu") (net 13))
 (segment (start 150.2625 130.61) (end 152.615 130.61) (width 0.25) (layer "F.Cu") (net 13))
 (segment (start 159.06172 124.16328) (end 159.06172 122.016341) (width 0.25) (layer "F.Cu") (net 13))
 (segment (start 159.06172 122.016341) (end 158.637025 121.591646) (width 0.25) (layer "F.Cu") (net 13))
 (segment (start 157.48 121.92) (end 156.975 121.92) (width 0.25) (layer "F.Cu") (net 13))
 (segment (start 156.565 121.51) (end 155.14 121.51) (width 0.25) (layer "F.Cu") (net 13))
 (segment (start 156.975 121.92) (end 156.565 121.51) (width 0.25) (layer "F.Cu") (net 13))
 (segment (start 152.615 130.61) (end 159.06172 124.16328) (width 0.25) (layer "F.Cu") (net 13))
 (segment (start 141.515 124.952462) (end 141.515 123.967538) (width 0.25) (layer "F.Cu") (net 24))
 (segment (start 140.7125 133.01) (end 140.6375 132.935) (width 0.25) (layer "F.Cu") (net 24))
 (segment (start 144.805 123.66) (end 145.605 124.46) (width 0.25) (layer "F.Cu") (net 24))
 (segment (start 145.605 124.46) (end 145.6125 124.4675) (width 0.25) (layer "F.Cu") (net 24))
 (segment (start 140.6375 125.829962) (end 141.515 124.952462) (width 0.25) (layer "F.Cu") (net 24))
 (segment (start 145.605 124.46) (end 148.555 121.51) (width 0.25) (layer "F.Cu") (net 24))
 (segment (start 141.822538 123.66) (end 144.805 123.66) (width 0.25) (layer "F.Cu") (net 24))
 (segment (start 141.515 123.967538) (end 141.822538 123.66) (width 0.25) (layer "F.Cu") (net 24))
 (segment (start 145.605 124.46) (end 145.903543 124.758543) (width 0.25) (layer "F.Cu") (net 24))
 (segment (start 140.6375 132.935) (end 140.6375 125.829962) (width 0.25) (layer "F.Cu") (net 24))
 (segment (start 152.375088 121.51) (end 152.94 122.074912) (width 0.25) (layer "F.Cu") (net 24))
 (segment (start 148.555 121.51) (end 152.375088 121.51) (width 0.25) (layer "F.Cu") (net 24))
 (segment (start 141.7625 133.01) (end 140.7125 133.01) (width 0.25) (layer "F.Cu") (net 24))
 (segment (start 152.94 122.074912) (end 152.94 124.46) (width 0.25) (layer "F.Cu") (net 24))
 (segment (start 139.7 125.35) (end 140.59 124.46) (width 0.25) (layer "F.Cu") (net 27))
 (segment (start 134.62 125.35) (end 137.16 125.35) (width 0.25) (layer "F.Cu") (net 27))
 (segment (start 137.16 125.35) (end 139.7 125.35) (width 0.25) (layer "F.Cu") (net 27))
 (segment (start 137.16 131.8575) (end 137.16 125.35) (width 0.25) (layer "F.Cu") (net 27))
 (segment (start 140.7125 135.41) (end 137.16 131.8575) (width 0.25) (layer "F.Cu") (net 27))
 (segment (start 141.7625 135.41) (end 140.7125 135.41) (width 0.25) (layer "F.Cu") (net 27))
 (segment (start 141.6325 132.08) (end 141.7625 132.21) (width 0.25) (layer "F.Cu") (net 23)))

